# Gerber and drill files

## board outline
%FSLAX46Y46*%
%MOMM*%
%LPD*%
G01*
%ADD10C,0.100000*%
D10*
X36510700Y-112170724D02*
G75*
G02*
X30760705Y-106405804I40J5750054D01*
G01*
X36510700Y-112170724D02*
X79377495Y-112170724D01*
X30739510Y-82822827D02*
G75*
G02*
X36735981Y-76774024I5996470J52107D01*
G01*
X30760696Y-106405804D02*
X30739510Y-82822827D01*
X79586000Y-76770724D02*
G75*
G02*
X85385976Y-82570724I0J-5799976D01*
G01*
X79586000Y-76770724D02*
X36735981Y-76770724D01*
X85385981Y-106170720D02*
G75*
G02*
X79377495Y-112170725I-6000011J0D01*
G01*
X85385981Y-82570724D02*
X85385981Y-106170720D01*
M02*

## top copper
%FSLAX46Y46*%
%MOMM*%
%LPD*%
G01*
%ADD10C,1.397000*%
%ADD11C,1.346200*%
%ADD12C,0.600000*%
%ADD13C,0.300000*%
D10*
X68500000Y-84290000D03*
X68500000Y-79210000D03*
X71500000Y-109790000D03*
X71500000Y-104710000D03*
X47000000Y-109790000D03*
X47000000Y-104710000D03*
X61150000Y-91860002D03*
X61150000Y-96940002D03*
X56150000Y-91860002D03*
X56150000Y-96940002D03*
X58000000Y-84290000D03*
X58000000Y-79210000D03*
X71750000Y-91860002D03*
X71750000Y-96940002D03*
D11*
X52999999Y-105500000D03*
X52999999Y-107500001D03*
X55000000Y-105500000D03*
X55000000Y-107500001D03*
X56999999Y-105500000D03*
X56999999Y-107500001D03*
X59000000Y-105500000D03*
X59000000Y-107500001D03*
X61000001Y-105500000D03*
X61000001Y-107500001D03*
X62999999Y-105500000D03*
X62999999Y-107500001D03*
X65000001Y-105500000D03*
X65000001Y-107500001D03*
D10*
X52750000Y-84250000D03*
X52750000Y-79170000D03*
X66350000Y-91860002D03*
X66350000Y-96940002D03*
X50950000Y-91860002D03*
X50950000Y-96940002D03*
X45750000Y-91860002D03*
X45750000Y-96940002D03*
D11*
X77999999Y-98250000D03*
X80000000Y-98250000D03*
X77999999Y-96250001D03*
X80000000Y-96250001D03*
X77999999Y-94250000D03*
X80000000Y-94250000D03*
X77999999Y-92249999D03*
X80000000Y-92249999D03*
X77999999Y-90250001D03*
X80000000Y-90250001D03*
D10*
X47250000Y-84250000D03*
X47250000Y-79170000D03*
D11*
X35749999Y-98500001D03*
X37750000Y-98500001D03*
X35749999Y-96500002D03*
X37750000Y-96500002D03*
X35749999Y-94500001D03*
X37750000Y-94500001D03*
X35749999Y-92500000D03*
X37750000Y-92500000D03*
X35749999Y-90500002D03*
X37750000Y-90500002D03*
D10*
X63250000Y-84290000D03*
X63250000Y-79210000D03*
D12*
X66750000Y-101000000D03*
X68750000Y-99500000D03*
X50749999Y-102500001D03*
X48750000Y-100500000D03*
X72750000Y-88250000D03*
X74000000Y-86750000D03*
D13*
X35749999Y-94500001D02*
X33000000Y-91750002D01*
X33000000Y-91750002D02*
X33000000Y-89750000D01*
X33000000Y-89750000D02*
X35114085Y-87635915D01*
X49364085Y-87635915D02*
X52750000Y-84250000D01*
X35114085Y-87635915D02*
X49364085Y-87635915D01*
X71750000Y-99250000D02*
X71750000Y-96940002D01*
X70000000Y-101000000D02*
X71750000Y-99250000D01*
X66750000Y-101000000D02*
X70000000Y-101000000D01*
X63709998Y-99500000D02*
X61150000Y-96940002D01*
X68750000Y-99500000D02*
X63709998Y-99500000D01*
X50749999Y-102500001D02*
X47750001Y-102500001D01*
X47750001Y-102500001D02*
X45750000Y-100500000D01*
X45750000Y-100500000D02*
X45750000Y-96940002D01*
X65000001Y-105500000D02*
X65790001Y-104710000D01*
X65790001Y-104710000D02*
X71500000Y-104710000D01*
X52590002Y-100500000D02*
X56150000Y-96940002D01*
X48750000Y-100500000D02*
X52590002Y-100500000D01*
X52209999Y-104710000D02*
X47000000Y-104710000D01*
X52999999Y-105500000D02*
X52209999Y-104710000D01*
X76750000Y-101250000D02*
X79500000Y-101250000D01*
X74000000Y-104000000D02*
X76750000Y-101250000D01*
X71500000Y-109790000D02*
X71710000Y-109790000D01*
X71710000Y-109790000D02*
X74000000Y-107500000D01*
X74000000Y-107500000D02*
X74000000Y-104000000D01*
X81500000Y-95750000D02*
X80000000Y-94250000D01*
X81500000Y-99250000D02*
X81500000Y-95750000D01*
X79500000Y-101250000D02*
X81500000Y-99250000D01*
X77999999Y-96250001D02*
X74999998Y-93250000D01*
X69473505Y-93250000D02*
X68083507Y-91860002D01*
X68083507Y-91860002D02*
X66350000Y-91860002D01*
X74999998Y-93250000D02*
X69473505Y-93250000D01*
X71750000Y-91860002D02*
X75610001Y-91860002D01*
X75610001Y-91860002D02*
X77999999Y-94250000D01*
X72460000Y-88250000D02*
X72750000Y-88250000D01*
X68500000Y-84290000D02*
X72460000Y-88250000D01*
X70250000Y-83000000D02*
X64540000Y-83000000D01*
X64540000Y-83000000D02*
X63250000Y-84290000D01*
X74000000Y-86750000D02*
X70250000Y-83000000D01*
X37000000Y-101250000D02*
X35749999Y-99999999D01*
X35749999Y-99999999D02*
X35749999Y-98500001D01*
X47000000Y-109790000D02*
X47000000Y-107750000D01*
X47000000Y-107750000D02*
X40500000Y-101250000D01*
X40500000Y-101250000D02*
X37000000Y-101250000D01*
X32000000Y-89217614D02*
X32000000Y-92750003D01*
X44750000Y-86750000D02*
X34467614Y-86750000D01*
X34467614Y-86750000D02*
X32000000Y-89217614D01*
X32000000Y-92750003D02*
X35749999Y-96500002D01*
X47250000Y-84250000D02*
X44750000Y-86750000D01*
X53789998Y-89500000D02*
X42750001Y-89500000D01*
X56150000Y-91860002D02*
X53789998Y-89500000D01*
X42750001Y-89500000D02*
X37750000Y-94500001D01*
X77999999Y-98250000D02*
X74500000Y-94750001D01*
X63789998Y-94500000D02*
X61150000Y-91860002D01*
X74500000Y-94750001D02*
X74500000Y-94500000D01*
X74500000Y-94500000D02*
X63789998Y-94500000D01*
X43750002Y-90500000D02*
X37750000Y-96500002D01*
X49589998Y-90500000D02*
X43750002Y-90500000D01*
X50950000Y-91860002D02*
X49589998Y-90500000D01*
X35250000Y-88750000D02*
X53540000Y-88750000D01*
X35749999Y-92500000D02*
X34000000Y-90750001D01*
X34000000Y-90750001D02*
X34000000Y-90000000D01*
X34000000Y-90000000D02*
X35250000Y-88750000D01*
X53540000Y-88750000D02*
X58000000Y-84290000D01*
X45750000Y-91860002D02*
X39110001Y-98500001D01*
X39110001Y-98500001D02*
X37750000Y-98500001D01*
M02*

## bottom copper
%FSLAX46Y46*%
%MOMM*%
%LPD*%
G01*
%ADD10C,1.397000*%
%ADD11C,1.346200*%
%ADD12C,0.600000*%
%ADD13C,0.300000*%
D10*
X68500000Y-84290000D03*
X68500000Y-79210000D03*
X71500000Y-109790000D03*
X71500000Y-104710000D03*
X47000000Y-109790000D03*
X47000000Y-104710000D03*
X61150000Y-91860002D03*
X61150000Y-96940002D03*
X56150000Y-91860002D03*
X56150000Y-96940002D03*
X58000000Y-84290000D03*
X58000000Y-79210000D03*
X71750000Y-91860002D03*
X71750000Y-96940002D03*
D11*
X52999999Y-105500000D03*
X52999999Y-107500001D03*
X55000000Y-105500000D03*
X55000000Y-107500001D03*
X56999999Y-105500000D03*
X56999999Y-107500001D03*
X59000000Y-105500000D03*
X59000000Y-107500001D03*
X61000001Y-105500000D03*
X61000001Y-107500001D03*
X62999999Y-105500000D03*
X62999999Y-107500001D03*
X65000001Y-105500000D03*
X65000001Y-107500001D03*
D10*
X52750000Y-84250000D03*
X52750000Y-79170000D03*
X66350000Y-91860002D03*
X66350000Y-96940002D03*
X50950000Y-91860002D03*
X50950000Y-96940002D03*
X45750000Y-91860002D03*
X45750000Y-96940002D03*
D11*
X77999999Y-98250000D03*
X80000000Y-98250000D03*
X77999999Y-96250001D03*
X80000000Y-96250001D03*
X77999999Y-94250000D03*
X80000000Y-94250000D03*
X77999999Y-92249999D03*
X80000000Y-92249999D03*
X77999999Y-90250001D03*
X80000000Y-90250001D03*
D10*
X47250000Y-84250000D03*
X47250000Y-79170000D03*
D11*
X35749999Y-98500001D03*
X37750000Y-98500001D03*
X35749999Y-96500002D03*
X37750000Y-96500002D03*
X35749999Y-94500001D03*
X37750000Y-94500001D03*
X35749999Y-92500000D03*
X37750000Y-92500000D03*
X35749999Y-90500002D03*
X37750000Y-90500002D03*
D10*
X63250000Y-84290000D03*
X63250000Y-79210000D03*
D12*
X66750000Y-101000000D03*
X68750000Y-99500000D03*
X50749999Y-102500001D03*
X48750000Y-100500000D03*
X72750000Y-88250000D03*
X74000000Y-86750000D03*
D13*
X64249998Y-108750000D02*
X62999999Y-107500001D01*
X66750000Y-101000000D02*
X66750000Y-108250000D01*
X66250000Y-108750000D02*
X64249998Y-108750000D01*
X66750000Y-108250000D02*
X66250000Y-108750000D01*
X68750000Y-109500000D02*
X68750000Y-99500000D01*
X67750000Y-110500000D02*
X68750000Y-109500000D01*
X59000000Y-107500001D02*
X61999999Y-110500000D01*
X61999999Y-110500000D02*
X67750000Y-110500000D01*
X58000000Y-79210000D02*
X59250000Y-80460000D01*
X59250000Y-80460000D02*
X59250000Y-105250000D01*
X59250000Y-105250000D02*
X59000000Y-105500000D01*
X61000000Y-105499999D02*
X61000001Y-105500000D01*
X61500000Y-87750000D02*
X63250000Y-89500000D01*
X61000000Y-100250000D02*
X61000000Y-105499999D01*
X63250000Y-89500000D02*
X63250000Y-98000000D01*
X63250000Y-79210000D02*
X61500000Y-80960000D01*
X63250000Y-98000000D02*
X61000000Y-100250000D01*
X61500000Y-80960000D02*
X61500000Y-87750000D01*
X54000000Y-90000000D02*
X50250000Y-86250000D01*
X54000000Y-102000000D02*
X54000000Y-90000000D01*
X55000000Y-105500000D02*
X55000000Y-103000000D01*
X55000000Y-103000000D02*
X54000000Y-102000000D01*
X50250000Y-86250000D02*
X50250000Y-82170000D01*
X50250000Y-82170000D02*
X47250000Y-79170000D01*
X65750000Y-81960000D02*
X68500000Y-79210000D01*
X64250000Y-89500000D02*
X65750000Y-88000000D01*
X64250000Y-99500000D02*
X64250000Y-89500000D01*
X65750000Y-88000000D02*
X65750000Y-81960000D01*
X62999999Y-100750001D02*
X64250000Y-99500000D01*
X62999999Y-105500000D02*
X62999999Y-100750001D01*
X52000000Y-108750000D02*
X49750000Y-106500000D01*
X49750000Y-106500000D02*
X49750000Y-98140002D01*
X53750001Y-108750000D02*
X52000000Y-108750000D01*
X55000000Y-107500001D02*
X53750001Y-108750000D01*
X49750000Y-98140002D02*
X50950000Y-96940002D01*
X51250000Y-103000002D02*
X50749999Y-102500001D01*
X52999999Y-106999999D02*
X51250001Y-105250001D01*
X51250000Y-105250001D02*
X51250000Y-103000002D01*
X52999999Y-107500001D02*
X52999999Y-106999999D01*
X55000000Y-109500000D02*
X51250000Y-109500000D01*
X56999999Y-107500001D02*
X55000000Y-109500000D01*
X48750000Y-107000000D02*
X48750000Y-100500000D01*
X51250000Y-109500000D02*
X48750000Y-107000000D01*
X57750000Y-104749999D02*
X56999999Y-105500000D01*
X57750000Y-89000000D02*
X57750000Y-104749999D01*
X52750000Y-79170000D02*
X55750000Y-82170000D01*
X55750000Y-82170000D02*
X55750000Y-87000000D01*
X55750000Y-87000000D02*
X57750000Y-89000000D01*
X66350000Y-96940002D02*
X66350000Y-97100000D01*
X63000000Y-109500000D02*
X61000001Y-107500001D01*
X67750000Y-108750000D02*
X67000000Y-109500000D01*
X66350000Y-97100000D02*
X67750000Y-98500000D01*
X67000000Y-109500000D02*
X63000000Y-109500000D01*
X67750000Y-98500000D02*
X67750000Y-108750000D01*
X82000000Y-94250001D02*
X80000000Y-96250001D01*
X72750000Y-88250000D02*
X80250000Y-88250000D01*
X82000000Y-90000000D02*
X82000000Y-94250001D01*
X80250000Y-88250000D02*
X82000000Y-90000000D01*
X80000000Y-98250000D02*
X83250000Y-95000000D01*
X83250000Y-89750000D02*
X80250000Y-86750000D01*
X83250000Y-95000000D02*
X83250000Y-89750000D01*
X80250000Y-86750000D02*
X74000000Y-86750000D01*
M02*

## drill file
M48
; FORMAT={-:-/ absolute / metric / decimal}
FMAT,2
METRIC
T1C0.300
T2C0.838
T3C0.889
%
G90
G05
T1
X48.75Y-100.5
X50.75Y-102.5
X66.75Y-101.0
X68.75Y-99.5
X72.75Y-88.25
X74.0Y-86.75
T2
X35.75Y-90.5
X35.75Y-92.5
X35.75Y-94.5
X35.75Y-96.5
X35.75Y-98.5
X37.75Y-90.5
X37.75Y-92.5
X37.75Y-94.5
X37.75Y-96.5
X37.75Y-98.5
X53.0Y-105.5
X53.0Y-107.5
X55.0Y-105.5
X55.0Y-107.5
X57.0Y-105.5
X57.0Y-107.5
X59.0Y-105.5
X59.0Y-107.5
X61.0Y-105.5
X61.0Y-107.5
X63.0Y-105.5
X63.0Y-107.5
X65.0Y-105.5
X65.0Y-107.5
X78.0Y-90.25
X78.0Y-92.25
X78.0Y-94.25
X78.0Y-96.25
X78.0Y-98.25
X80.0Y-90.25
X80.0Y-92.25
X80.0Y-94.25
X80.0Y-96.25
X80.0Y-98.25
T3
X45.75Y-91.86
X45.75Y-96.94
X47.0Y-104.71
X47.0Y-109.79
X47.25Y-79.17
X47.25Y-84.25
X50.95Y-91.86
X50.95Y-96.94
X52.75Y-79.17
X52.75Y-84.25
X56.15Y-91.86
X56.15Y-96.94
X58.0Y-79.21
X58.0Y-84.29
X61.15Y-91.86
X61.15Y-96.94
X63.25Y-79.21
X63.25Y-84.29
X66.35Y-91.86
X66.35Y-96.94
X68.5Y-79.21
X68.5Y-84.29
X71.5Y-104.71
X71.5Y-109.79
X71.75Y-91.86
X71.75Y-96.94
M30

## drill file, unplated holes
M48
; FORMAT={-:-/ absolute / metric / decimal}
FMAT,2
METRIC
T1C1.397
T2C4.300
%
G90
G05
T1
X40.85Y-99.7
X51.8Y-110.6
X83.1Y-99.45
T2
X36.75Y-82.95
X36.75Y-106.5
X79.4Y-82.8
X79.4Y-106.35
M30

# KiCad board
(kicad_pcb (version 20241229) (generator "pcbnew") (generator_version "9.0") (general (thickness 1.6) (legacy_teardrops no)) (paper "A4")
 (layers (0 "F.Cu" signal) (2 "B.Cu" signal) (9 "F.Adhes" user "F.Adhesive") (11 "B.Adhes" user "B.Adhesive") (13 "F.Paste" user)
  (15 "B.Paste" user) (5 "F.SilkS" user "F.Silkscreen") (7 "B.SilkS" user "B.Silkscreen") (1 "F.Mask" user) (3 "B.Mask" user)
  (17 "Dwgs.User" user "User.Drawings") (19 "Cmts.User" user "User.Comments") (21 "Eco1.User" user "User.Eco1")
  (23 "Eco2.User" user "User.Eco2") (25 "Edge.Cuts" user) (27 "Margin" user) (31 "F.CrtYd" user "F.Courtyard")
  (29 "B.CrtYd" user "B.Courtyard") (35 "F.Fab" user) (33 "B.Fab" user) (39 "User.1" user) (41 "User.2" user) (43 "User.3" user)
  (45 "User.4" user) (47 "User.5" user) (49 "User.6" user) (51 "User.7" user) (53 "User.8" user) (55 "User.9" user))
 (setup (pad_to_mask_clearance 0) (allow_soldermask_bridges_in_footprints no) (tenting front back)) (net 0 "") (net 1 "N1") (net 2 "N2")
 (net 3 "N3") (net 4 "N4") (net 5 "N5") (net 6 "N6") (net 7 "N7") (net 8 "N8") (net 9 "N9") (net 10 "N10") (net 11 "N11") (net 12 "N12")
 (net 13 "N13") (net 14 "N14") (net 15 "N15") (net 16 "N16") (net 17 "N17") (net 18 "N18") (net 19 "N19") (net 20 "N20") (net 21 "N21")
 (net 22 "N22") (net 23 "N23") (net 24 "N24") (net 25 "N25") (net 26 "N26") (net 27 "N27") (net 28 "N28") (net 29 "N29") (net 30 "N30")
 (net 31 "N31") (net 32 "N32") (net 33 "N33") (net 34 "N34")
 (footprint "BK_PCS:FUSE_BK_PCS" (layer "F.Cu") (at 68.5 81.75 90)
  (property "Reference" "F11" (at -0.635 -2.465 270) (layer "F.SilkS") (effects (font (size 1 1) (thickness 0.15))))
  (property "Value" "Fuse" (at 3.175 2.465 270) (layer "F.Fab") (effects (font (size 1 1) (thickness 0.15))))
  (pad "1" thru_hole circle (at -2.54 0 90) (size 1.397 1.397) (drill 0.889) (layers "*.Cu" "*.Mask") (remove_unused_layers no) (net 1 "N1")
   (solder_mask_margin 0.102))
  (pad "2" thru_hole circle (at 2.54 0 90) (size 1.397 1.397) (drill 0.889) (layers "*.Cu" "*.Mask") (remove_unused_layers no) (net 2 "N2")
   (solder_mask_margin 0.102)))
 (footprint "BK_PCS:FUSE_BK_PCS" (layer "F.Cu") (at 71.5 107.25 90)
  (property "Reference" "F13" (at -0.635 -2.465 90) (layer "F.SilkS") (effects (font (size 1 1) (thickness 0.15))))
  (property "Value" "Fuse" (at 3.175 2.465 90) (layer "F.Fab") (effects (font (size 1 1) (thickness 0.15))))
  (pad "1" thru_hole circle (at -2.54 0 90) (size 1.397 1.397) (drill 0.889) (layers "*.Cu" "*.Mask") (remove_unused_layers no) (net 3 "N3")
   (solder_mask_margin 0.102))
  (pad "2" thru_hole circle (at 2.54 0 90) (size 1.397 1.397) (drill 0.889) (layers "*.Cu" "*.Mask") (remove_unused_layers no) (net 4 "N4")
   (solder_mask_margin 0.102)))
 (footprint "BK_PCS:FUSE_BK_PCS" (layer "F.Cu") (at 47 107.25 90)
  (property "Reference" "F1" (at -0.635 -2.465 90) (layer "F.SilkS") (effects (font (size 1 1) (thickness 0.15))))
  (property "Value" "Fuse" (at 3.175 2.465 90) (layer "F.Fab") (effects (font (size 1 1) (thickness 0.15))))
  (pad "1" thru_hole circle (at -2.54 0 90) (size 1.397 1.397) (drill 0.889) (layers "*.Cu" "*.Mask") (remove_unused_layers no) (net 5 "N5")
   (solder_mask_margin 0.102))
  (pad "2" thru_hole circle (at 2.54 0 90) (size 1.397 1.397) (drill 0.889) (layers "*.Cu" "*.Mask") (remove_unused_layers no) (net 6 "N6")
   (solder_mask_margin 0.102)))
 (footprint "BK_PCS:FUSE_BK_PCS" (layer "F.Cu") (at 61.15 94.400002 -90)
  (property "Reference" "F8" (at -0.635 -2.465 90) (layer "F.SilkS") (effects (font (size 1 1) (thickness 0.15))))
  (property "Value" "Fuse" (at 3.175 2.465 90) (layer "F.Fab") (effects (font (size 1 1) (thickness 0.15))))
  (pad "1" thru_hole circle (at -2.54 0 270) (size 1.397 1.397) (drill 0.889) (layers "*.Cu" "*.Mask") (remove_unused_layers no)
   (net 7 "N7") (solder_mask_margin 0.102))
  (pad "2" thru_hole circle (at 2.54 0 270) (size 1.397 1.397) (drill 0.889) (layers "*.Cu" "*.Mask") (remove_unused_layers no) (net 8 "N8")
   (solder_mask_margin 0.102)))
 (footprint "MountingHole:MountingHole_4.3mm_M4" (layer "F.Cu") (at 36.75 106.5)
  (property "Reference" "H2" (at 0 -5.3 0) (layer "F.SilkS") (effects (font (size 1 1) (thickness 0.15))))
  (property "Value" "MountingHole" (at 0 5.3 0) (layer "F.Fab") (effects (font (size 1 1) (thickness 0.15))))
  (pad "" np_thru_hole circle (at 0 0) (size 4.3 4.3) (drill 4.3) (layers "*.Cu" "*.Mask")))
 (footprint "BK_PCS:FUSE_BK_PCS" (layer "F.Cu") (at 56.15 94.400002 -90)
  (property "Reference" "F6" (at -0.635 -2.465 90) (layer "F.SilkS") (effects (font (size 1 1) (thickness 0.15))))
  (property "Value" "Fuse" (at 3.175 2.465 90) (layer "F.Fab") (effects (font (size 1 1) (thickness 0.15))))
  (pad "1" thru_hole circle (at -2.54 0 270) (size 1.397 1.397) (drill 0.889) (layers "*.Cu" "*.Mask") (remove_unused_layers no)
   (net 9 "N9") (solder_mask_margin 0.102))
  (pad "2" thru_hole circle (at 2.54 0 270) (size 1.397 1.397) (drill 0.889) (layers "*.Cu" "*.Mask") (remove_unused_layers no)
   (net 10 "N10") (solder_mask_margin 0.102)))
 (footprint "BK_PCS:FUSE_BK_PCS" (layer "F.Cu") (at 58 81.75 90)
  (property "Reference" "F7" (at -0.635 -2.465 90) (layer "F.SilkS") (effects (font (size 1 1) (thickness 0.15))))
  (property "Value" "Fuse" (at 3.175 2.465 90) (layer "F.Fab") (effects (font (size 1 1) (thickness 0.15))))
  (pad "1" thru_hole circle (at -2.54 0 90) (size 1.397 1.397) (drill 0.889) (layers "*.Cu" "*.Mask") (remove_unused_layers no)
   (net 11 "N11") (solder_mask_margin 0.102))
  (pad "2" thru_hole circle (at 2.54 0 90) (size 1.397 1.397) (drill 0.889) (layers "*.Cu" "*.Mask") (remove_unused_layers no)
   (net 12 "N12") (solder_mask_margin 0.102)))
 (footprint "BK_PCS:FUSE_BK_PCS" (layer "F.Cu") (at 71.75 94.400002 -90)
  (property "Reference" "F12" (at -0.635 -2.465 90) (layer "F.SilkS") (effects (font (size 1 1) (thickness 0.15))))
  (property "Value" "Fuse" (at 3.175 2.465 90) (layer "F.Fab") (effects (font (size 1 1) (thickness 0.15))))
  (pad "1" thru_hole circle (at -2.54 0 270) (size 1.397 1.397) (drill 0.889) (layers "*.Cu" "*.Mask") (remove_unused_layers no)
   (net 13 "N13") (solder_mask_margin 0.102))
  (pad "2" thru_hole circle (at 2.54 0 270) (size 1.397 1.397) (drill 0.889) (layers "*.Cu" "*.Mask") (remove_unused_layers no)
   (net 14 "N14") (solder_mask_margin 0.102)))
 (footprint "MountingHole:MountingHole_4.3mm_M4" (layer "F.Cu") (at 36.75 82.95)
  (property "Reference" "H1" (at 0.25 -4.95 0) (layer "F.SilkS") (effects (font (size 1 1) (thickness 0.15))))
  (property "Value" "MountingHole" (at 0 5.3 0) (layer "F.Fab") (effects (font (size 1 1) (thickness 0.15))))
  (pad "" np_thru_hole circle (at 0 0) (size 4.3 4.3) (drill 4.3) (layers "*.Cu" "*.Mask")))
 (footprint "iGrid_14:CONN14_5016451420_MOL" (layer "F.Cu") (at 52.999999 105.5)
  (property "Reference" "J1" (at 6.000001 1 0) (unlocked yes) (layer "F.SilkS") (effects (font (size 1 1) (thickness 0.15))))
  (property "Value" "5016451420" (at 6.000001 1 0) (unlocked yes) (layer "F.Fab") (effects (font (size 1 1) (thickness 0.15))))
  (pad "" np_thru_hole circle (at -1.2 5.099999) (size 1.397 1.397) (drill 1.397) (layers "*.Cu" "*.Mask"))
  (pad "1" thru_hole circle (at 0 0) (size 1.3462 1.3462) (drill 0.8382) (layers "*.Cu" "*.Mask") (remove_unused_layers no) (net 6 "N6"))
  (pad "2" thru_hole circle (at 0 2.000001) (size 1.3462 1.3462) (drill 0.8382) (layers "*.Cu" "*.Mask") (remove_unused_layers no)
   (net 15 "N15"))
  (pad "3" thru_hole circle (at 2.000001 0) (size 1.3462 1.3462) (drill 0.8382) (layers "*.Cu" "*.Mask") (remove_unused_layers no)
   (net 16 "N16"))
  (pad "4" thru_hole circle (at 2.000001 2.000001) (size 1.3462 1.3462) (drill 0.8382) (layers "*.Cu" "*.Mask") (remove_unused_layers no)
   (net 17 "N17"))
  (pad "5" thru_hole circle (at 4 0) (size 1.3462 1.3462) (drill 0.8382) (layers "*.Cu" "*.Mask") (remove_unused_layers no) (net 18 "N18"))
  (pad "6" thru_hole circle (at 4 2.000001) (size 1.3462 1.3462) (drill 0.8382) (layers "*.Cu" "*.Mask") (remove_unused_layers no)
   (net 10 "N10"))
  (pad "7" thru_hole circle (at 6.000001 0) (size 1.3462 1.3462) (drill 0.8382) (layers "*.Cu" "*.Mask") (remove_unused_layers no)
   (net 12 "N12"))
  (pad "8" thru_hole circle (at 6.000001 2.000001) (size 1.3462 1.3462) (drill 0.8382) (layers "*.Cu" "*.Mask") (remove_unused_layers no)
   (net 8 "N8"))
  (pad "9" thru_hole circle (at 8.000002 0) (size 1.3462 1.3462) (drill 0.8382) (layers "*.Cu" "*.Mask") (remove_unused_layers no)
   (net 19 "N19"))
  (pad "10" thru_hole circle (at 8.000002 2.000001) (size 1.3462 1.3462) (drill 0.8382) (layers "*.Cu" "*.Mask") (remove_unused_layers no)
   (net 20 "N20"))
  (pad "11" thru_hole circle (at 10 0) (size 1.3462 1.3462) (drill 0.8382) (layers "*.Cu" "*.Mask") (remove_unused_layers no) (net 2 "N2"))
  (pad "12" thru_hole circle (at 10 2.000001) (size 1.3462 1.3462) (drill 0.8382) (layers "*.Cu" "*.Mask") (remove_unused_layers no)
   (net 14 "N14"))
  (pad "13" thru_hole circle (at 12.000002 0) (size 1.3462 1.3462) (drill 0.8382) (layers "*.Cu" "*.Mask") (remove_unused_layers no)
   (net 4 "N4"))
  (pad "14" thru_hole circle (at 12.000002 2.000001) (size 1.3462 1.3462) (drill 0.8382) (layers "*.Cu" "*.Mask") (remove_unused_layers no)
   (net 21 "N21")))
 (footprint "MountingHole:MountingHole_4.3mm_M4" (layer "F.Cu") (at 79.4 82.8)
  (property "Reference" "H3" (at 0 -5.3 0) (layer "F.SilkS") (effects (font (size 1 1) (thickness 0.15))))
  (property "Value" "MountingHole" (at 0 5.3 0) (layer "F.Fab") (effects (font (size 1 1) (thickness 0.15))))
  (pad "" np_thru_hole circle (at 0 0) (size 4.3 4.3) (drill 4.3) (layers "*.Cu" "*.Mask")))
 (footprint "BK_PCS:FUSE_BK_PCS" (layer "F.Cu") (at 52.75 81.71 90)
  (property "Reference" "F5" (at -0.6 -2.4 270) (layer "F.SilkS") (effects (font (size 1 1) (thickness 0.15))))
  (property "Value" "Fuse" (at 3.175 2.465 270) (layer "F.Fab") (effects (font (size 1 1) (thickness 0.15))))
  (pad "1" thru_hole circle (at -2.54 0 90) (size 1.397 1.397) (drill 0.889) (layers "*.Cu" "*.Mask") (remove_unused_layers no)
   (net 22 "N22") (solder_mask_margin 0.102))
  (pad "2" thru_hole circle (at 2.54 0 90) (size 1.397 1.397) (drill 0.889) (layers "*.Cu" "*.Mask") (remove_unused_layers no)
   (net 18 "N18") (solder_mask_margin 0.102)))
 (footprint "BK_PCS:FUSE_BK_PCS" (layer "F.Cu") (at 66.35 94.400002 -90)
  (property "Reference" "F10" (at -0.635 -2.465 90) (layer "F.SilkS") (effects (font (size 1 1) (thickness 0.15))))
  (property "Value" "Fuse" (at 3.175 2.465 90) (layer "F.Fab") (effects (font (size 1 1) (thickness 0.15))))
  (pad "1" thru_hole circle (at -2.54 0 270) (size 1.397 1.397) (drill 0.889) (layers "*.Cu" "*.Mask") (remove_unused_layers no)
   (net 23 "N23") (solder_mask_margin 0.102))
  (pad "2" thru_hole circle (at 2.54 0 270) (size 1.397 1.397) (drill 0.889) (layers "*.Cu" "*.Mask") (remove_unused_layers no)
   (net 20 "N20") (solder_mask_margin 0.102)))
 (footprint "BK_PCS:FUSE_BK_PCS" (layer "F.Cu") (at 50.95 94.400002 -90)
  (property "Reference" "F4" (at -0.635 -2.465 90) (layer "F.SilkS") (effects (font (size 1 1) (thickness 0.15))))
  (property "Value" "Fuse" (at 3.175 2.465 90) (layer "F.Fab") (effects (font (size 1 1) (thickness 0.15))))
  (pad "1" thru_hole circle (at -2.54 0 270) (size 1.397 1.397) (drill 0.889) (layers "*.Cu" "*.Mask") (remove_unused_layers no)
   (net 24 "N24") (solder_mask_margin 0.102))
  (pad "2" thru_hole circle (at 2.54 0 270) (size 1.397 1.397) (drill 0.889) (layers "*.Cu" "*.Mask") (remove_unused_layers no)
   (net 17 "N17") (solder_mask_margin 0.102)))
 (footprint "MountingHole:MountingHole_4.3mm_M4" (layer "F.Cu") (at 79.4 106.35)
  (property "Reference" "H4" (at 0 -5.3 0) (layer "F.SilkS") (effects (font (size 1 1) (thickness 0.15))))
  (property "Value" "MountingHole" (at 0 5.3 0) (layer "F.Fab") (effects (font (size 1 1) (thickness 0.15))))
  (pad "" np_thru_hole circle (at 0 0) (size 4.3 4.3) (drill 4.3) (layers "*.Cu" "*.Mask")))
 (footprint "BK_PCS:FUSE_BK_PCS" (layer "F.Cu") (at 45.75 94.400002 -90)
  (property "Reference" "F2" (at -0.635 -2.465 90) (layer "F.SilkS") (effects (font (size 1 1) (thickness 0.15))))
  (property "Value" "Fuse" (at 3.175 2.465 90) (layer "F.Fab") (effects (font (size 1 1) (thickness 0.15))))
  (pad "1" thru_hole circle (at -2.54 0 270) (size 1.397 1.397) (drill 0.889) (layers "*.Cu" "*.Mask") (remove_unused_layers no)
   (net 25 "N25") (solder_mask_margin 0.102))
  (pad "2" thru_hole circle (at 2.54 0 270) (size 1.397 1.397) (drill 0.889) (layers "*.Cu" "*.Mask") (remove_unused_layers no)
   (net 15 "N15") (solder_mask_margin 0.102)))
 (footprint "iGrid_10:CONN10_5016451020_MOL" (layer "F.Cu") (at 77.999999 98.25 90)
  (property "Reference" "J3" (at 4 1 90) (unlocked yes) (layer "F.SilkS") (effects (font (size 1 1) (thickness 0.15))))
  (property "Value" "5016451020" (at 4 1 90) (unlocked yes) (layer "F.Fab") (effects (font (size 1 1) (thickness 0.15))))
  (pad "" np_thru_hole circle (at -1.2 5.099999 90) (size 1.397 1.397) (drill 1.397) (layers "*.Cu" "*.Mask"))
  (pad "1" thru_hole circle (at 0 0 90) (size 1.3462 1.3462) (drill 0.8382) (layers "*.Cu" "*.Mask") (remove_unused_layers no) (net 7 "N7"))
  (pad "2" thru_hole circle (at 0 2.000001 90) (size 1.3462 1.3462) (drill 0.8382) (layers "*.Cu" "*.Mask") (remove_unused_layers no)
   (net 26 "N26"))
  (pad "3" thru_hole circle (at 1.999999 0 90) (size 1.3462 1.3462) (drill 0.8382) (layers "*.Cu" "*.Mask") (remove_unused_layers no)
   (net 23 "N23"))
  (pad "4" thru_hole circle (at 1.999999 2.000001 90) (size 1.3462 1.3462) (drill 0.8382) (layers "*.Cu" "*.Mask") (remove_unused_layers no)
   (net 1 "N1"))
  (pad "5" thru_hole circle (at 4 0 90) (size 1.3462 1.3462) (drill 0.8382) (layers "*.Cu" "*.Mask") (remove_unused_layers no)
   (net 13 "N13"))
  (pad "6" thru_hole circle (at 4 2.000001 90) (size 1.3462 1.3462) (drill 0.8382) (layers "*.Cu" "*.Mask") (remove_unused_layers no)
   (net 3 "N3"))
  (pad "7" thru_hole circle (at 6.000001 0 90) (size 1.3462 1.3462) (drill 0.8382) (layers "*.Cu" "*.Mask") (remove_unused_layers no)
   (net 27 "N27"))
  (pad "8" thru_hole circle (at 6.000001 2.000001 90) (size 1.3462 1.3462) (drill 0.8382) (layers "*.Cu" "*.Mask") (remove_unused_layers no)
   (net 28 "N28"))
  (pad "9" thru_hole circle (at 7.999999 0 90) (size 1.3462 1.3462) (drill 0.8382) (layers "*.Cu" "*.Mask") (remove_unused_layers no)
   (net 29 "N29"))
  (pad "10" thru_hole circle (at 7.999999 2.000001 90) (size 1.3462 1.3462) (drill 0.8382) (layers "*.Cu" "*.Mask")
   (remove_unused_layers no) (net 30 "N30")))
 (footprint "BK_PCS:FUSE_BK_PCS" (layer "F.Cu") (at 47.25 81.71 90)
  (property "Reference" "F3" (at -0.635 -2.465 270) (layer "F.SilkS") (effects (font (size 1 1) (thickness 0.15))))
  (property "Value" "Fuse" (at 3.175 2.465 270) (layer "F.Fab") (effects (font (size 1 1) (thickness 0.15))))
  (pad "1" thru_hole circle (at -2.54 0 90) (size 1.397 1.397) (drill 0.889) (layers "*.Cu" "*.Mask") (remove_unused_layers no)
   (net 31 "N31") (solder_mask_margin 0.102))
  (pad "2" thru_hole circle (at 2.54 0 90) (size 1.397 1.397) (drill 0.889) (layers "*.Cu" "*.Mask") (remove_unused_layers no)
   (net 16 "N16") (solder_mask_margin 0.102)))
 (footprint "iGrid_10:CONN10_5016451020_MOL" (layer "F.Cu") (at 35.749999 98.500001 90)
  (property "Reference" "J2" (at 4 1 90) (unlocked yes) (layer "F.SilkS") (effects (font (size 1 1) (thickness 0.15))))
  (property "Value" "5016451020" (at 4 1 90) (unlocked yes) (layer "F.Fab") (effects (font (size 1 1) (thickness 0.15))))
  (pad "" np_thru_hole circle (at -1.2 5.099999 90) (size 1.397 1.397) (drill 1.397) (layers "*.Cu" "*.Mask"))
  (pad "1" thru_hole circle (at 0 0 90) (size 1.3462 1.3462) (drill 0.8382) (layers "*.Cu" "*.Mask") (remove_unused_layers no) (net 5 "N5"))
  (pad "2" thru_hole circle (at 0 2.000001 90) (size 1.3462 1.3462) (drill 0.8382) (layers "*.Cu" "*.Mask") (remove_unused_layers no)
   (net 25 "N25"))
  (pad "3" thru_hole circle (at 1.999999 0 90) (size 1.3462 1.3462) (drill 0.8382) (layers "*.Cu" "*.Mask") (remove_unused_layers no)
   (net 31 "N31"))
  (pad "4" thru_hole circle (at 1.999999 2.000001 90) (size 1.3462 1.3462) (drill 0.8382) (layers "*.Cu" "*.Mask") (remove_unused_layers no)
   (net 24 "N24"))
  (pad "5" thru_hole circle (at 4 0 90) (size 1.3462 1.3462) (drill 0.8382) (layers "*.Cu" "*.Mask") (remove_unused_layers no)
   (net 22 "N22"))
  (pad "6" thru_hole circle (at 4 2.000001 90) (size 1.3462 1.3462) (drill 0.8382) (layers "*.Cu" "*.Mask") (remove_unused_layers no)
   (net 9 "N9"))
  (pad "7" thru_hole circle (at 6.000001 0 90) (size 1.3462 1.3462) (drill 0.8382) (layers "*.Cu" "*.Mask") (remove_unused_layers no)
   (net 11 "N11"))
  (pad "8" thru_hole circle (at 6.000001 2.000001 90) (size 1.3462 1.3462) (drill 0.8382) (layers "*.Cu" "*.Mask") (remove_unused_layers no)
   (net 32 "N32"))
  (pad "9" thru_hole circle (at 7.999999 0 90) (size 1.3462 1.3462) (drill 0.8382) (layers "*.Cu" "*.Mask") (remove_unused_layers no)
   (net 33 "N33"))
  (pad "10" thru_hole circle (at 7.999999 2.000001 90) (size 1.3462 1.3462) (drill 0.8382) (layers "*.Cu" "*.Mask")
   (remove_unused_layers no) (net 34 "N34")))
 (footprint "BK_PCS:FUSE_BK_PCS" (layer "F.Cu") (at 63.25 81.75 90)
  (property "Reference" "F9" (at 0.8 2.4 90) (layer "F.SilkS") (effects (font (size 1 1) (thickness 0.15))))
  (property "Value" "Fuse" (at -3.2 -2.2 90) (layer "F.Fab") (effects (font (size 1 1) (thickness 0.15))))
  (pad "1" thru_hole circle (at -2.54 0 90) (size 1.397 1.397) (drill 0.889) (layers "*.Cu" "*.Mask") (remove_unused_layers no)
   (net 26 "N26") (solder_mask_margin 0.102))
  (pad "2" thru_hole circle (at 2.54 0 90) (size 1.397 1.397) (drill 0.889) (layers "*.Cu" "*.Mask") (remove_unused_layers no)
   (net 19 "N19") (solder_mask_margin 0.102)))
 (gr_arc (start 36.5107 112.170724) (mid 32.444847 110.486588) (end 30.760696 106.405804) (stroke (width 0.1) (type solid))
  (layer "Edge.Cuts"))
 (gr_line (start 36.5107 112.170724) (end 79.377495 112.170724) (stroke (width 0.1) (type solid)) (layer "Edge.Cuts"))
 (gr_arc (start 30.73951 82.822827) (mid 32.495676 78.530419) (end 36.735981 76.774027) (stroke (width 0.1) (type solid))
  (layer "Edge.Cuts"))
 (gr_line (start 30.760696 106.405804) (end 30.73951 82.822827) (stroke (width 0.1) (type solid)) (layer "Edge.Cuts"))
 (gr_arc (start 79.586 76.770724) (mid 83.6872 78.469505) (end 85.385981 82.570724) (stroke (width 0.1) (type solid)) (layer "Edge.Cuts"))
 (gr_line (start 79.586 76.770724) (end 36.735981 76.770724) (stroke (width 0.1) (type solid)) (layer "Edge.Cuts"))
 (gr_arc (start 85.385981 106.17072) (mid 83.628622 110.413365) (end 79.377495 112.170724) (stroke (width 0.1) (type solid))
  (layer "Edge.Cuts"))
 (gr_line (start 85.385981 82.570724) (end 85.385981 106.17072) (stroke (width 0.1) (type solid)) (layer "Edge.Cuts"))
 (segment (start 71.75 99.25) (end 71.75 96.940002) (width 0.3) (layer "F.Cu") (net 14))
 (segment (start 70 101) (end 71.75 99.25) (width 0.3) (layer "F.Cu") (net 14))
 (segment (start 66.75 101) (end 70 101) (width 0.3) (layer "F.Cu") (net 14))
 (via (at 66.75 101) (size 0.6) (drill 0.3) (layers "F.Cu" "B.Cu") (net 14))
 (segment (start 64.249998 108.75) (end 62.999999 107.500001) (width 0.3) (layer "B.Cu") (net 14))
 (segment (start 66.75 101) (end 66.75 108.25) (width 0.3) (layer "B.Cu") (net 14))
 (segment (start 66.25 108.75) (end 64.249998 108.75) (width 0.3) (layer "B.Cu") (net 14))
 (segment (start 66.75 108.25) (end 66.25 108.75) (width 0.3) (layer "B.Cu") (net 14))
 (segment (start 63.709998 99.5) (end 61.15 96.940002) (width 0.3) (layer "F.Cu") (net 8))
 (segment (start 68.75 99.5) (end 63.709998 99.5) (width 0.3) (layer "F.Cu") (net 8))
 (via (at 68.75 99.5) (size 0.6) (drill 0.3) (layers "F.Cu" "B.Cu") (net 8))
 (segment (start 68.75 109.5) (end 68.75 99.5) (width 0.3) (layer "B.Cu") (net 8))
 (segment (start 67.75 110.5) (end 68.75 109.5) (width 0.3) (layer "B.Cu") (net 8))
 (segment (start 59 107.500001) (end 61.999999 110.5) (width 0.3) (layer "B.Cu") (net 8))
 (segment (start 61.999999 110.5) (end 67.75 110.5) (width 0.3) (layer "B.Cu") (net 8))
 (segment (start 58 79.21) (end 59.25 80.46) (width 0.3) (layer "B.Cu") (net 12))
 (segment (start 59.25 80.46) (end 59.25 105.25) (width 0.3) (layer "B.Cu") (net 12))
 (segment (start 59.25 105.25) (end 59 105.5) (width 0.3) (layer "B.Cu") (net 12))
 (segment (start 61 105.499999) (end 61.000001 105.5) (width 0.3) (layer "B.Cu") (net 19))
 (segment (start 61.5 87.75) (end 63.25 89.5) (width 0.3) (layer "B.Cu") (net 19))
 (segment (start 61 100.25) (end 61 105.499999) (width 0.3) (layer "B.Cu") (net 19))
 (segment (start 63.25 89.5) (end 63.25 98) (width 0.3) (layer "B.Cu") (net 19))
 (segment (start 63.25 79.21) (end 61.5 80.96) (width 0.3) (layer "B.Cu") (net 19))
 (segment (start 63.25 98) (end 61 100.25) (width 0.3) (layer "B.Cu") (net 19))
 (segment (start 61.5 80.96) (end 61.5 87.75) (width 0.3) (layer "B.Cu") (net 19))
 (segment (start 54 90) (end 50.25 86.25) (width 0.3) (layer "B.Cu") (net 16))
 (segment (start 54 102) (end 54 90) (width 0.3) (layer "B.Cu") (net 16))
 (segment (start 55 105.5) (end 55 103) (width 0.3) (layer "B.Cu") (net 16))
 (segment (start 55 103) (end 54 102) (width 0.3) (layer "B.Cu") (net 16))
 (segment (start 50.25 86.25) (end 50.25 82.17) (width 0.3) (layer "B.Cu") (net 16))
 (segment (start 50.25 82.17) (end 47.25 79.17) (width 0.3) (layer "B.Cu") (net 16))
 (segment (start 65.75 81.96) (end 68.5 79.21) (width 0.3) (layer "B.Cu") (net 2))
 (segment (start 64.25 89.5) (end 65.75 88) (width 0.3) (layer "B.Cu") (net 2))
 (segment (start 64.25 99.5) (end 64.25 89.5) (width 0.3) (layer "B.Cu") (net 2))
 (segment (start 65.75 88) (end 65.75 81.96) (width 0.3) (layer "B.Cu") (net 2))
 (segment (start 62.999999 100.750001) (end 64.25 99.5) (width 0.3) (layer "B.Cu") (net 2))
 (segment (start 62.999999 105.5) (end 62.999999 100.750001) (width 0.3) (layer "B.Cu") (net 2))
 (segment (start 52 108.75) (end 49.75 106.5) (width 0.3) (layer "B.Cu") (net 17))
 (segment (start 49.75 106.5) (end 49.75 98.140002) (width 0.3) (layer "B.Cu") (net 17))
 (segment (start 53.750001 108.75) (end 52 108.75) (width 0.3) (layer "B.Cu") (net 17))
 (segment (start 55 107.500001) (end 53.750001 108.75) (width 0.3) (layer "B.Cu") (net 17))
 (segment (start 49.75 98.140002) (end 50.95 96.940002) (width 0.3) (layer "B.Cu") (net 17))
 (segment (start 50.749999 102.500001) (end 47.750001 102.500001) (width 0.3) (layer "F.Cu") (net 15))
 (segment (start 47.750001 102.500001) (end 45.75 100.5) (width 0.3) (layer "F.Cu") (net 15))
 (segment (start 45.75 100.5) (end 45.75 96.940002) (width 0.3) (layer "F.Cu") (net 15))
 (via (at 50.749999 102.500001) (size 0.6) (drill 0.3) (layers "F.Cu" "B.Cu") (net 15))
 (segment (start 51.25 103.000002) (end 50.749999 102.500001) (width 0.3) (layer "B.Cu") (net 15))
 (segment (start 52.999999 106.999999) (end 51.250001 105.250001) (width 0.3) (layer "B.Cu") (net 15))
 (segment (start 51.25 105.250001) (end 51.25 103.000002) (width 0.3) (layer "B.Cu") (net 15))
 (segment (start 52.999999 107.500001) (end 52.999999 106.999999) (width 0.3) (layer "B.Cu") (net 15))
 (segment (start 65.000001 105.5) (end 65.790001 104.71) (width 0.3) (layer "F.Cu") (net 4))
 (segment (start 65.790001 104.71) (end 71.5 104.71) (width 0.3) (layer "F.Cu") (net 4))
 (segment (start 52.590002 100.5) (end 56.15 96.940002) (width 0.3) (layer "F.Cu") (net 10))
 (segment (start 48.75 100.5) (end 52.590002 100.5) (width 0.3) (layer "F.Cu") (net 10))
 (via (at 48.75 100.5) (size 0.6) (drill 0.3) (layers "F.Cu" "B.Cu") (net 10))
 (segment (start 55 109.5) (end 51.25 109.5) (width 0.3) (layer "B.Cu") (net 10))
 (segment (start 56.999999 107.500001) (end 55 109.5) (width 0.3) (layer "B.Cu") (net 10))
 (segment (start 48.75 107) (end 48.75 100.5) (width 0.3) (layer "B.Cu") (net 10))
 (segment (start 51.25 109.5) (end 48.75 107) (width 0.3) (layer "B.Cu") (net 10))
 (segment (start 52.209999 104.71) (end 47 104.71) (width 0.3) (layer "F.Cu") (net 6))
 (segment (start 52.999999 105.5) (end 52.209999 104.71) (width 0.3) (layer "F.Cu") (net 6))
 (segment (start 57.75 104.749999) (end 56.999999 105.5) (width 0.3) (layer "B.Cu") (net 18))
 (segment (start 57.75 89) (end 57.75 104.749999) (width 0.3) (layer "B.Cu") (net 18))
 (segment (start 52.75 79.17) (end 55.75 82.17) (width 0.3) (layer "B.Cu") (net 18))
 (segment (start 55.75 82.17) (end 55.75 87) (width 0.3) (layer "B.Cu") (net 18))
 (segment (start 55.75 87) (end 57.75 89) (width 0.3) (layer "B.Cu") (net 18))
 (segment (start 66.35 96.940002) (end 66.35 97.1) (width 0.3) (layer "B.Cu") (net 20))
 (segment (start 63 109.5) (end 61.000001 107.500001) (width 0.3) (layer "B.Cu") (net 20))
 (segment (start 67.75 108.75) (end 67 109.5) (width 0.3) (layer "B.Cu") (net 20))
 (segment (start 66.35 97.1) (end 67.75 98.5) (width 0.3) (layer "B.Cu") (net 20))
 (segment (start 67 109.5) (end 63 109.5) (width 0.3) (layer "B.Cu") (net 20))
 (segment (start 67.75 98.5) (end 67.75 108.75) (width 0.3) (layer "B.Cu") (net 20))
 (segment (start 76.75 101.25) (end 79.5 101.25) (width 0.3) (layer "F.Cu") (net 3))
 (segment (start 74 104) (end 76.75 101.25) (width 0.3) (layer "F.Cu") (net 3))
 (segment (start 71.5 109.79) (end 71.71 109.79) (width 0.3) (layer "F.Cu") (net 3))
 (segment (start 71.71 109.79) (end 74 107.5) (width 0.3) (layer "F.Cu") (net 3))
 (segment (start 74 107.5) (end 74 104) (width 0.3) (layer "F.Cu") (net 3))
 (segment (start 81.5 95.75) (end 80 94.25) (width 0.3) (layer "F.Cu") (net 3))
 (segment (start 81.5 99.25) (end 81.5 95.75) (width 0.3) (layer "F.Cu") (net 3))
 (segment (start 79.5 101.25) (end 81.5 99.25) (width 0.3) (layer "F.Cu") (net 3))
 (segment (start 77.999999 96.250001) (end 74.999998 93.25) (width 0.3) (layer "F.Cu") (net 23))
 (segment (start 69.473505 93.25) (end 68.083507 91.860002) (width 0.3) (layer "F.Cu") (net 23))
 (segment (start 68.083507 91.860002) (end 66.35 91.860002) (width 0.3) (layer "F.Cu") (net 23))
 (segment (start 74.999998 93.25) (end 69.473505 93.25) (width 0.3) (layer "F.Cu") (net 23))
 (segment (start 71.75 91.860002) (end 75.610001 91.860002) (width 0.3) (layer "F.Cu") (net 13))
 (segment (start 75.610001 91.860002) (end 77.999999 94.25) (width 0.3) (layer "F.Cu") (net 13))
 (segment (start 72.46 88.25) (end 72.75 88.25) (width 0.3) (layer "F.Cu") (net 1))
 (segment (start 68.5 84.29) (end 72.46 88.25) (width 0.3) (layer "F.Cu") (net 1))
 (via (at 72.75 88.25) (size 0.6) (drill 0.3) (layers "F.Cu" "B.Cu") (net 1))
 (segment (start 82 94.250001) (end 80 96.250001) (width 0.3) (layer "B.Cu") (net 1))
 (segment (start 72.75 88.25) (end 80.25 88.25) (width 0.3) (layer "B.Cu") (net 1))
 (segment (start 82 90) (end 82 94.250001) (width 0.3) (layer "B.Cu") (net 1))
 (segment (start 80.25 88.25) (end 82 90) (width 0.3) (layer "B.Cu") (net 1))
 (segment (start 70.25 83) (end 64.54 83) (width 0.3) (layer "F.Cu") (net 26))
 (segment (start 64.54 83) (end 63.25 84.29) (width 0.3) (layer "F.Cu") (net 26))
 (segment (start 74 86.75) (end 70.25 83) (width 0.3) (layer "F.Cu") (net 26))
 (via (at 74 86.75) (size 0.6) (drill 0.3) (layers "F.Cu" "B.Cu") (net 26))
 (segment (start 80 98.25) (end 83.25 95) (width 0.3) (layer "B.Cu") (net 26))
 (segment (start 83.25 89.75) (end 80.25 86.75) (width 0.3) (layer "B.Cu") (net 26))
 (segment (start 83.25 95) (end 83.25 89.75) (width 0.3) (layer "B.Cu") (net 26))
 (segment (start 80.25 86.75) (end 74 86.75) (width 0.3) (layer "B.Cu") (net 26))
 (segment (start 37 101.25) (end 35.749999 99.999999) (width 0.3) (layer "F.Cu") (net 5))
 (segment (start 35.749999 99.999999) (end 35.749999 98.500001) (width 0.3) (layer "F.Cu") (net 5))
 (segment (start 47 109.79) (end 47 107.75) (width 0.3) (layer "F.Cu") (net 5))
 (segment (start 47 107.75) (end 40.5 101.25) (width 0.3) (layer "F.Cu") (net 5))
 (segment (start 40.5 101.25) (end 37 101.25) (width 0.3) (layer "F.Cu") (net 5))
 (segment (start 35.749999 94.500001) (end 33 91.750002) (width 0.3) (layer "F.Cu") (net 22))
 (segment (start 33 89.75) (end 35.114085 87.635915) (width 0.3) (layer "F.Cu") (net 22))
 (segment (start 33 91.750002) (end 33 89.75) (width 0.3) (layer "F.Cu") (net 22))
 (segment (start 49.364085 87.635915) (end 52.75 84.25) (width 0.3) (layer "F.Cu") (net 22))
 (segment (start 35.114085 87.635915) (end 49.364085 87.635915) (width 0.3) (layer "F.Cu") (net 22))
 (segment (start 32 89.217614) (end 32 92.750003) (width 0.3) (layer "F.Cu") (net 31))
 (segment (start 44.75 86.75) (end 34.467614 86.75) (width 0.3) (layer "F.Cu") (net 31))
 (segment (start 34.467614 86.75) (end 32 89.217614) (width 0.3) (layer "F.Cu") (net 31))
 (segment (start 32 92.750003) (end 35.749999 96.500002) (width 0.3) (layer "F.Cu") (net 31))
 (segment (start 47.25 84.25) (end 44.75 86.75) (width 0.3) (layer "F.Cu") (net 31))
 (segment (start 53.789998 89.5) (end 42.750001 89.5) (width 0.3) (layer "F.Cu") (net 9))
 (segment (start 56.15 91.860002) (end 53.789998 89.5) (width 0.3) (layer "F.Cu") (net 9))
 (segment (start 42.750001 89.5) (end 37.75 94.500001) (width 0.3) (layer "F.Cu") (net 9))
 (segment (start 77.999999 98.25) (end 74.5 94.750001) (width 0.3) (layer "F.Cu") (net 7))
 (segment (start 63.789998 94.5) (end 61.15 91.860002) (width 0.3) (layer "F.Cu") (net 7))
 (segment (start 74.5 94.750001) (end 74.5 94.5) (width 0.3) (layer "F.Cu") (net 7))
 (segment (start 74.5 94.5) (end 63.789998 94.5) (width 0.3) (layer "F.Cu") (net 7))
 (segment (start 43.750002 90.5) (end 37.75 96.500002) (width 0.3) (layer "F.Cu") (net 24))
 (segment (start 49.589998 90.5) (end 43.750002 90.5) (width 0.3) (layer "F.Cu") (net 24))
 (segment (start 50.95 91.860002) (end 49.589998 90.5) (width 0.3) (layer "F.Cu") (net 24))
 (segment (start 35.25 88.75) (end 53.54 88.75) (width 0.3) (layer "F.Cu") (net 11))
 (segment (start 35.749999 92.5) (end 34 90.750001) (width 0.3) (layer "F.Cu") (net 11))
 (segment (start 34 90.750001) (end 34 90) (width 0.3) (layer "F.Cu") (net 11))
 (segment (start 34 90) (end 35.25 88.75) (width 0.3) (layer "F.Cu") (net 11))
 (segment (start 53.54 88.75) (end 58 84.29) (width 0.3) (layer "F.Cu") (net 11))
 (segment (start 45.75 91.860002) (end 39.110001 98.500001) (width 0.3) (layer "F.Cu") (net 25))
 (segment (start 39.110001 98.500001) (end 37.75 98.500001) (width 0.3) (layer "F.Cu") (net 25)))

